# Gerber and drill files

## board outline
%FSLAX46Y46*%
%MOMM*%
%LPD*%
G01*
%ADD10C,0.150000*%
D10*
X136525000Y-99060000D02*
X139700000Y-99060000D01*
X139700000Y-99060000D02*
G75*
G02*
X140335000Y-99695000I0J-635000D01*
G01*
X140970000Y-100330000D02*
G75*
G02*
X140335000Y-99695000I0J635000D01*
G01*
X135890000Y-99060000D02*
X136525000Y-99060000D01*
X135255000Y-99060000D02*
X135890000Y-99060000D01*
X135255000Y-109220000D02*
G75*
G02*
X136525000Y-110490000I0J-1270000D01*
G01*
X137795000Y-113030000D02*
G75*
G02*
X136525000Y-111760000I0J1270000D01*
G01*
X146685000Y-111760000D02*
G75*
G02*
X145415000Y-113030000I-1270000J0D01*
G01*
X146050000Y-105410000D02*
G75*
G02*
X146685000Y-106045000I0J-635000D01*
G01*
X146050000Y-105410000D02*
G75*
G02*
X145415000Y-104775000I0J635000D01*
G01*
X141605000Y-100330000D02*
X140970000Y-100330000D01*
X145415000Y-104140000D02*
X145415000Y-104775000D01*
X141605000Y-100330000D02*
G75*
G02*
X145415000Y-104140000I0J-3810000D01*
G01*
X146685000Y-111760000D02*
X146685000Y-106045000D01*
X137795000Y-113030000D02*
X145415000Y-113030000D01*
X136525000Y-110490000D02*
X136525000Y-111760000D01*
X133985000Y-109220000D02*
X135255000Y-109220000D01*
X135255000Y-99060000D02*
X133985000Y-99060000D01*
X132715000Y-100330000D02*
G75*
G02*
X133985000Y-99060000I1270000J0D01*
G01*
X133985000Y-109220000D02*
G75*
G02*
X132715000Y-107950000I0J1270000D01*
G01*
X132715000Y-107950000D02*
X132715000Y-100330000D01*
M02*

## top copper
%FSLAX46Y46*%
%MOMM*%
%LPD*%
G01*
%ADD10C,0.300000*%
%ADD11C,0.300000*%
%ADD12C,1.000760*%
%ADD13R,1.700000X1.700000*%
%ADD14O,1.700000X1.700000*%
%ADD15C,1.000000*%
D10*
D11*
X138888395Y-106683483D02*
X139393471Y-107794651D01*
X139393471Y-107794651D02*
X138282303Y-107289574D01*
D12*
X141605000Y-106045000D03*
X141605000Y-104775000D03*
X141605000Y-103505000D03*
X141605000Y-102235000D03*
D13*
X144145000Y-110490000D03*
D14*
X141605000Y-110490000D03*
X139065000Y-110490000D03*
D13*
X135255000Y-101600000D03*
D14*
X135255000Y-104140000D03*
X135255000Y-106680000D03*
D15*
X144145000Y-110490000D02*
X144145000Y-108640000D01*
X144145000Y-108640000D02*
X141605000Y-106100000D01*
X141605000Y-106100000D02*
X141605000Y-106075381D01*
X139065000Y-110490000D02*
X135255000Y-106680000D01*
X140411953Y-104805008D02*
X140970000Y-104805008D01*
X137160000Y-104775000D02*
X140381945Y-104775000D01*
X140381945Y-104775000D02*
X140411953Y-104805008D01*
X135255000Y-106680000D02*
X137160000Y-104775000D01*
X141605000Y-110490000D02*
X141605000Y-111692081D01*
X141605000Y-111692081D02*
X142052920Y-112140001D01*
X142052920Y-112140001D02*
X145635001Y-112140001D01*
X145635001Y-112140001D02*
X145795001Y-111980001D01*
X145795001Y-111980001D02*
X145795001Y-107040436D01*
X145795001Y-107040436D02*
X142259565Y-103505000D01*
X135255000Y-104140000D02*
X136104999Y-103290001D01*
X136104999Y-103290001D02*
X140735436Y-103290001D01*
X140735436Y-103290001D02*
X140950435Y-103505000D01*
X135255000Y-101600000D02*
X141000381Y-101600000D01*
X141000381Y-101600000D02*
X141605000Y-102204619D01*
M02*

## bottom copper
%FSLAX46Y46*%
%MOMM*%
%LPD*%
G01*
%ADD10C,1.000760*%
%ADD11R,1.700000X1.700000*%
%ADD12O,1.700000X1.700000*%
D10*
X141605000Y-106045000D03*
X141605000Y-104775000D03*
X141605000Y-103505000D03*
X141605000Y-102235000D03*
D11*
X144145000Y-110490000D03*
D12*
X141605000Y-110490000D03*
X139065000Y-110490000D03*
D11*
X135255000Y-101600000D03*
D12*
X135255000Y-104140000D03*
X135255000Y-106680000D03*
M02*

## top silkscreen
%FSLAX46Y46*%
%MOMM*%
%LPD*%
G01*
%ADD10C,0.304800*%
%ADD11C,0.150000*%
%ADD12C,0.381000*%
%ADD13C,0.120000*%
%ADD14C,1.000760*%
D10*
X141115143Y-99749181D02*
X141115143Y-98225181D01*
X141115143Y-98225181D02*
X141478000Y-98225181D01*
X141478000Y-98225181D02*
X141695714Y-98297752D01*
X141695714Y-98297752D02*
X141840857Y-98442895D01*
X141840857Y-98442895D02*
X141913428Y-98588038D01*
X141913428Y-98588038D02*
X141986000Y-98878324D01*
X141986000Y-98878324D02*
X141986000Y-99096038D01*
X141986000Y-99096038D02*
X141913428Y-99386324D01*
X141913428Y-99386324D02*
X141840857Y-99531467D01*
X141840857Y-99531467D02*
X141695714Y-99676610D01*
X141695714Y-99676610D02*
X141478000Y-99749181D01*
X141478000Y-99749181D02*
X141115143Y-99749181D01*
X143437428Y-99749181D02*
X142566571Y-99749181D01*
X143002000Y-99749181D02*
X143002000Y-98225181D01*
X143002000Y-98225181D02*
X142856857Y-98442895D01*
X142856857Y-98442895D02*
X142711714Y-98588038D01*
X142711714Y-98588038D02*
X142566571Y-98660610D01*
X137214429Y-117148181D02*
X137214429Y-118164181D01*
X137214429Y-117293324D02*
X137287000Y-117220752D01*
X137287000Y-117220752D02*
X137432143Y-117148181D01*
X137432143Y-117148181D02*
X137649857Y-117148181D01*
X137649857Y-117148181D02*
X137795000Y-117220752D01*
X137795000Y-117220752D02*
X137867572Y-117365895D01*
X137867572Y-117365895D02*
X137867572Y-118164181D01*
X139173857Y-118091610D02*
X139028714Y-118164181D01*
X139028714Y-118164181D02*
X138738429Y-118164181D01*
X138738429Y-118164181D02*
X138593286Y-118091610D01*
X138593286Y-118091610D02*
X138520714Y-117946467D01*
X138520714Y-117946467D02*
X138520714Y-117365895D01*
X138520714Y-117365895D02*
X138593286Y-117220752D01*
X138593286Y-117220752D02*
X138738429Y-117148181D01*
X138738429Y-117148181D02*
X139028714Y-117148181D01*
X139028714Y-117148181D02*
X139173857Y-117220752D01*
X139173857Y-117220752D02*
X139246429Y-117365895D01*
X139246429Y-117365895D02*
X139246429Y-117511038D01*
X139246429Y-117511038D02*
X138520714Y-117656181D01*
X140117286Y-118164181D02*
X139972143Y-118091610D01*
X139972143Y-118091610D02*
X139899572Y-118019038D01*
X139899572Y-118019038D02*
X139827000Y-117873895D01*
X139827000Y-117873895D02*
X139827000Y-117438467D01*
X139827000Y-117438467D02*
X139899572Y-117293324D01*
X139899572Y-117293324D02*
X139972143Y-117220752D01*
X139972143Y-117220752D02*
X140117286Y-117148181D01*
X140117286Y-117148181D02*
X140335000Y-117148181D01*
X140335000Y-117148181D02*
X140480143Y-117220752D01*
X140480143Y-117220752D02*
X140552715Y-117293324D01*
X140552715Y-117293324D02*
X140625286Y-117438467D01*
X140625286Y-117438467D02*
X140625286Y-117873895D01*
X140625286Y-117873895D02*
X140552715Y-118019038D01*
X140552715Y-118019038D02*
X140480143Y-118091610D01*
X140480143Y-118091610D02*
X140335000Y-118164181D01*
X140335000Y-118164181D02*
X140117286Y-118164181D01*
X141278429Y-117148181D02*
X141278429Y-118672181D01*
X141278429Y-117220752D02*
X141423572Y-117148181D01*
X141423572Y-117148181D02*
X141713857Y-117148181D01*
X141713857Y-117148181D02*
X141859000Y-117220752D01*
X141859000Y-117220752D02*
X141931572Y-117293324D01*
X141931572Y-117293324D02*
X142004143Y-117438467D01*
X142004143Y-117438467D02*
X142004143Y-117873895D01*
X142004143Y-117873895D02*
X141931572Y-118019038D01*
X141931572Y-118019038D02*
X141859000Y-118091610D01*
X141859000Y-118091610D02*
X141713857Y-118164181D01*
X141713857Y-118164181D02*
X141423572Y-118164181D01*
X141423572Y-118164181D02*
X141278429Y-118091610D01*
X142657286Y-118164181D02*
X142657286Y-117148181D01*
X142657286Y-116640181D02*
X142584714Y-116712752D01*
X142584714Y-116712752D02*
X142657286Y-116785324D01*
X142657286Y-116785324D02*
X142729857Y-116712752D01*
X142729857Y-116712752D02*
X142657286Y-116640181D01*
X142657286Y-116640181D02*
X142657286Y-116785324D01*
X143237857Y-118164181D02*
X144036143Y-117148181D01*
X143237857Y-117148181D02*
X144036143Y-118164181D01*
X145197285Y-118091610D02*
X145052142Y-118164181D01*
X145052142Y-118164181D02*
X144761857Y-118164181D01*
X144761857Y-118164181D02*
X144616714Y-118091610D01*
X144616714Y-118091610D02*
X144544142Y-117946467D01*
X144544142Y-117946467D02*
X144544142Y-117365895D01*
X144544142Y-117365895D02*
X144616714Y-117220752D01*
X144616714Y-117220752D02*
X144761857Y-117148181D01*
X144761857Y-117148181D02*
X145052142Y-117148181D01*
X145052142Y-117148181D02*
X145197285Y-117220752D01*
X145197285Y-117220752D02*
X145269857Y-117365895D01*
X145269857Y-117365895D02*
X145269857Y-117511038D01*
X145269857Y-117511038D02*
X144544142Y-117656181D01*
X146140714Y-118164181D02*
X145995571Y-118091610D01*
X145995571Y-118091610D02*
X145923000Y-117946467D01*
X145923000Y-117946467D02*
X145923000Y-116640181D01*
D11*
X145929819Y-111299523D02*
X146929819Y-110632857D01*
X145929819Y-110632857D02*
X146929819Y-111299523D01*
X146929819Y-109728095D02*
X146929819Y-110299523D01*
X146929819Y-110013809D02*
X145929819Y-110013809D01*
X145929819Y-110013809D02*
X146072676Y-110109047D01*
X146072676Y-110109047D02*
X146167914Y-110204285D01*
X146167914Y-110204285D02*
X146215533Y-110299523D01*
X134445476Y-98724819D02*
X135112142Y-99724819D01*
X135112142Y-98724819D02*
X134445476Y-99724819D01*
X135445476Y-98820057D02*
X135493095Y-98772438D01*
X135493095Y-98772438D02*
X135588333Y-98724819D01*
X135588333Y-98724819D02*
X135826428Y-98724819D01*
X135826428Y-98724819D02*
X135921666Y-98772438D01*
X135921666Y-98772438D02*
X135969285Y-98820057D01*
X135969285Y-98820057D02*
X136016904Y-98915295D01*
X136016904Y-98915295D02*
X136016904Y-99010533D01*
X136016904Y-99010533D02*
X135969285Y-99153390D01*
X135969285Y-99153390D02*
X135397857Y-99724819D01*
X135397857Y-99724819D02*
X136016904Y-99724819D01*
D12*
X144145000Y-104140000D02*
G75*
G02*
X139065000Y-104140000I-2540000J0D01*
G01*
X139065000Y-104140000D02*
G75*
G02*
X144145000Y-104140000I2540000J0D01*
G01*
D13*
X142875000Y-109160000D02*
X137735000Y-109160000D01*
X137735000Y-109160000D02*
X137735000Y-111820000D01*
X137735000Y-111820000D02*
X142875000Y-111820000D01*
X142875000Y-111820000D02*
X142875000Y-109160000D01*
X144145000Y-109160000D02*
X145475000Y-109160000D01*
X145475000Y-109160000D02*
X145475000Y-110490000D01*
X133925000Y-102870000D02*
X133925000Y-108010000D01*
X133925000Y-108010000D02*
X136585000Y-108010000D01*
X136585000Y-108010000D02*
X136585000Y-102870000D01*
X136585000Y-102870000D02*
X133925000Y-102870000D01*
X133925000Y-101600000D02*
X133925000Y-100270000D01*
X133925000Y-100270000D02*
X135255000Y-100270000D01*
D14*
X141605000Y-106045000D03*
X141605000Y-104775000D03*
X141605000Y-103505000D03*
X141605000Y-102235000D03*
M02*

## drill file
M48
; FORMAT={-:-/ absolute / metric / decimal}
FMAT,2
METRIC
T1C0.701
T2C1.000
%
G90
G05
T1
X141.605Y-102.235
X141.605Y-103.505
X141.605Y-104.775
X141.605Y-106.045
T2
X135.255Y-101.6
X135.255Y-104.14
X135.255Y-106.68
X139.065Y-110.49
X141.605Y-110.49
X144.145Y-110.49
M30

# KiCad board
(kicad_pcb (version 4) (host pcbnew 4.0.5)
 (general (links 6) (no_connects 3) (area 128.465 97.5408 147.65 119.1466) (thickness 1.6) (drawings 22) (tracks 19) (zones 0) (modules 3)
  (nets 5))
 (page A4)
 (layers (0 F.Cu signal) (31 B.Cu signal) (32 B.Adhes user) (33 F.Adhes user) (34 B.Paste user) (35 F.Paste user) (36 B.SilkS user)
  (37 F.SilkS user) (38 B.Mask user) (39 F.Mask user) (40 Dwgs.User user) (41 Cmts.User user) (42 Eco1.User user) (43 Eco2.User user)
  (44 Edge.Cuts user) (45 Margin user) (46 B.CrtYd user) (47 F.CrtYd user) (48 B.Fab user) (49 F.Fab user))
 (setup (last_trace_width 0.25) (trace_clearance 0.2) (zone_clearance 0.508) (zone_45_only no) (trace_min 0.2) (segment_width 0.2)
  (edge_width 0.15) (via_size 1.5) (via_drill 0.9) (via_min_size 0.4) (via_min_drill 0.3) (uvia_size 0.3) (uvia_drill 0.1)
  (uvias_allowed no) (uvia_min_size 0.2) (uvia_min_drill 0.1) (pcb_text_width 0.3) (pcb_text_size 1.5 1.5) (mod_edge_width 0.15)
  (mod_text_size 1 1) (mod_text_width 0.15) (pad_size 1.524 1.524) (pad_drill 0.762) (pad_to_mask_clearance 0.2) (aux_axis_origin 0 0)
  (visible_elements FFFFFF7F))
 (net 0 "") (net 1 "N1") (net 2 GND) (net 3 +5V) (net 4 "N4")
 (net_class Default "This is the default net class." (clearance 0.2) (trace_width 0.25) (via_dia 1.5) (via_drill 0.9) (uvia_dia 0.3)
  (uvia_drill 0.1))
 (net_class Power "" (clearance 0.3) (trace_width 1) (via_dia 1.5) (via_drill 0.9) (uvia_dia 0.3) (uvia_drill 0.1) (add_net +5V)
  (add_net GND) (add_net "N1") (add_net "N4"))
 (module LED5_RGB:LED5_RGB (layer F.Cu) (at 141.605 104.14 90)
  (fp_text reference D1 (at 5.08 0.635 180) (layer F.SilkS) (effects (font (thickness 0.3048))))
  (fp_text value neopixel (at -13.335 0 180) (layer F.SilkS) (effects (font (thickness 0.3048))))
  (fp_circle (center 0 0) (end 2.54 0) (layer F.SilkS) (width 0.381))
  (pad 1 thru_hole circle (at -1.905 0 90) (size 1.00076 1.00076) (drill 0.70104) (layers *.Cu *.Mask F.SilkS) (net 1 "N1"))
  (pad 2 thru_hole circle (at -0.635 0 90) (size 1.00076 1.00076) (drill 0.70104) (layers *.Cu *.Mask F.SilkS) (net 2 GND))
  (pad 3 thru_hole circle (at 0.635 0 90) (size 1.00076 1.00076) (drill 0.70104) (layers *.Cu *.Mask F.SilkS) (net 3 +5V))
  (pad 4 thru_hole circle (at 1.905 0 90) (size 1.00076 1.00076) (drill 0.70104) (layers *.Cu *.Mask F.SilkS) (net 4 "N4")))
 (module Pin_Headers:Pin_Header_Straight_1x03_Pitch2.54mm (layer F.Cu) (at 144.145 110.49 270)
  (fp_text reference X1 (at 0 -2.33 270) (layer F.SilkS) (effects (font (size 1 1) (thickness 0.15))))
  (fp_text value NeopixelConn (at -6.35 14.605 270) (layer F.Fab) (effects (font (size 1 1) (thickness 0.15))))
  (fp_line (start -1.33 1.27) (end -1.33 6.41) (layer F.SilkS) (width 0.12))
  (fp_line (start -1.33 6.41) (end 1.33 6.41) (layer F.SilkS) (width 0.12))
  (fp_line (start 1.33 6.41) (end 1.33 1.27) (layer F.SilkS) (width 0.12))
  (fp_line (start 1.33 1.27) (end -1.33 1.27) (layer F.SilkS) (width 0.12))
  (fp_line (start -1.33 0) (end -1.33 -1.33) (layer F.SilkS) (width 0.12))
  (fp_line (start -1.33 -1.33) (end 0 -1.33) (layer F.SilkS) (width 0.12))
  (pad 1 thru_hole rect (at 0 0 270) (size 1.7 1.7) (drill 1) (layers *.Cu *.Mask) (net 1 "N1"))
  (pad 2 thru_hole oval (at 0 2.54 270) (size 1.7 1.7) (drill 1) (layers *.Cu *.Mask) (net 3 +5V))
  (pad 3 thru_hole oval (at 0 5.08 270) (size 1.7 1.7) (drill 1) (layers *.Cu *.Mask) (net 2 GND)))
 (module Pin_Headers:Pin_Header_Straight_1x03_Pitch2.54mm (layer F.Cu) (at 135.255 101.6)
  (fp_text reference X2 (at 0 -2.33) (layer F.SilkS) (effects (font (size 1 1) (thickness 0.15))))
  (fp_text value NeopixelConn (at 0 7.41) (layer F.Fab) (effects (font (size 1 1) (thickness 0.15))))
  (fp_line (start -1.33 1.27) (end -1.33 6.41) (layer F.SilkS) (width 0.12))
  (fp_line (start -1.33 6.41) (end 1.33 6.41) (layer F.SilkS) (width 0.12))
  (fp_line (start 1.33 6.41) (end 1.33 1.27) (layer F.SilkS) (width 0.12))
  (fp_line (start 1.33 1.27) (end -1.33 1.27) (layer F.SilkS) (width 0.12))
  (fp_line (start -1.33 0) (end -1.33 -1.33) (layer F.SilkS) (width 0.12))
  (fp_line (start -1.33 -1.33) (end 0 -1.33) (layer F.SilkS) (width 0.12))
  (pad 1 thru_hole rect (at 0 0) (size 1.7 1.7) (drill 1) (layers *.Cu *.Mask) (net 4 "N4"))
  (pad 2 thru_hole oval (at 0 2.54) (size 1.7 1.7) (drill 1) (layers *.Cu *.Mask) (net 3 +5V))
  (pad 3 thru_hole oval (at 0 5.08) (size 1.7 1.7) (drill 1) (layers *.Cu *.Mask) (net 2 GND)))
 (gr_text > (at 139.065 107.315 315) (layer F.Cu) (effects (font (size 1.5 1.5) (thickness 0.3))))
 (gr_line (start 136.525 99.06) (end 139.7 99.06) (layer Edge.Cuts) (width 0.15))
 (gr_arc (start 139.7 99.695) (end 139.7 99.06) (angle 90) (layer Edge.Cuts) (width 0.15))
 (gr_arc (start 140.97 99.695) (end 140.97 100.33) (angle 90) (layer Edge.Cuts) (width 0.15))
 (gr_line (start 135.89 99.06) (end 136.525 99.06) (layer Edge.Cuts) (width 0.15))
 (gr_line (start 135.255 99.06) (end 135.89 99.06) (layer Edge.Cuts) (width 0.15))
 (gr_arc (start 135.255 110.49) (end 135.255 109.22) (angle 90) (layer Edge.Cuts) (width 0.15))
 (gr_arc (start 137.795 111.76) (end 137.795 113.03) (angle 90) (layer Edge.Cuts) (width 0.15))
 (gr_arc (start 145.415 111.76) (end 146.685 111.76) (angle 90) (layer Edge.Cuts) (width 0.15))
 (gr_arc (start 146.05 106.045) (end 146.05 105.41) (angle 90) (layer Edge.Cuts) (width 0.15))
 (gr_arc (start 146.05 104.775) (end 146.05 105.41) (angle 90) (layer Edge.Cuts) (width 0.15))
 (gr_line (start 141.605 100.33) (end 140.97 100.33) (layer Edge.Cuts) (width 0.15))
 (gr_line (start 145.415 104.14) (end 145.415 104.775) (layer Edge.Cuts) (width 0.15))
 (gr_arc (start 141.605 104.14) (end 141.605 100.33) (angle 90) (layer Edge.Cuts) (width 0.15))
 (gr_line (start 146.685 111.76) (end 146.685 106.045) (layer Edge.Cuts) (width 0.15))
 (gr_line (start 137.795 113.03) (end 145.415 113.03) (layer Edge.Cuts) (width 0.15))
 (gr_line (start 136.525 110.49) (end 136.525 111.76) (layer Edge.Cuts) (width 0.15))
 (gr_line (start 133.985 109.22) (end 135.255 109.22) (layer Edge.Cuts) (width 0.15))
 (gr_line (start 135.255 99.06) (end 133.985 99.06) (layer Edge.Cuts) (width 0.15))
 (gr_arc (start 133.985 100.33) (end 132.715 100.33) (angle 90) (layer Edge.Cuts) (width 0.15))
 (gr_arc (start 133.985 107.95) (end 133.985 109.22) (angle 90) (layer Edge.Cuts) (width 0.15))
 (gr_line (start 132.715 107.95) (end 132.715 100.33) (layer Edge.Cuts) (width 0.15))
 (segment (start 144.145 110.49) (end 144.145 108.64) (width 1) (layer F.Cu) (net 1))
 (segment (start 144.145 108.64) (end 141.605 106.1) (width 1) (layer F.Cu) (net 1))
 (segment (start 141.605 106.1) (end 141.605 106.075381) (width 1) (layer F.Cu) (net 1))
 (segment (start 139.065 110.49) (end 135.255 106.68) (width 1) (layer F.Cu) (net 2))
 (segment (start 140.411953 104.805008) (end 140.97 104.805008) (width 1) (layer F.Cu) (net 2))
 (segment (start 137.16 104.775) (end 140.381945 104.775) (width 1) (layer F.Cu) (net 2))
 (segment (start 140.381945 104.775) (end 140.411953 104.805008) (width 1) (layer F.Cu) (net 2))
 (segment (start 135.255 106.68) (end 137.16 104.775) (width 1) (layer F.Cu) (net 2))
 (segment (start 141.605 110.49) (end 141.605 111.692081) (width 1) (layer F.Cu) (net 3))
 (segment (start 141.605 111.692081) (end 142.05292 112.140001) (width 1) (layer F.Cu) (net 3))
 (segment (start 142.05292 112.140001) (end 145.635001 112.140001) (width 1) (layer F.Cu) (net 3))
 (segment (start 145.635001 112.140001) (end 145.795001 111.980001) (width 1) (layer F.Cu) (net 3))
 (segment (start 145.795001 111.980001) (end 145.795001 107.040436) (width 1) (layer F.Cu) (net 3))
 (segment (start 145.795001 107.040436) (end 142.259565 103.505) (width 1) (layer F.Cu) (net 3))
 (segment (start 135.255 104.14) (end 136.104999 103.290001) (width 1) (layer F.Cu) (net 3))
 (segment (start 136.104999 103.290001) (end 140.735436 103.290001) (width 1) (layer F.Cu) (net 3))
 (segment (start 140.735436 103.290001) (end 140.950435 103.505) (width 1) (layer F.Cu) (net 3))
 (segment (start 135.255 101.6) (end 141.000381 101.6) (width 1) (layer F.Cu) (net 4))
 (segment (start 141.000381 101.6) (end 141.605 102.204619) (width 1) (layer F.Cu) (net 4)))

